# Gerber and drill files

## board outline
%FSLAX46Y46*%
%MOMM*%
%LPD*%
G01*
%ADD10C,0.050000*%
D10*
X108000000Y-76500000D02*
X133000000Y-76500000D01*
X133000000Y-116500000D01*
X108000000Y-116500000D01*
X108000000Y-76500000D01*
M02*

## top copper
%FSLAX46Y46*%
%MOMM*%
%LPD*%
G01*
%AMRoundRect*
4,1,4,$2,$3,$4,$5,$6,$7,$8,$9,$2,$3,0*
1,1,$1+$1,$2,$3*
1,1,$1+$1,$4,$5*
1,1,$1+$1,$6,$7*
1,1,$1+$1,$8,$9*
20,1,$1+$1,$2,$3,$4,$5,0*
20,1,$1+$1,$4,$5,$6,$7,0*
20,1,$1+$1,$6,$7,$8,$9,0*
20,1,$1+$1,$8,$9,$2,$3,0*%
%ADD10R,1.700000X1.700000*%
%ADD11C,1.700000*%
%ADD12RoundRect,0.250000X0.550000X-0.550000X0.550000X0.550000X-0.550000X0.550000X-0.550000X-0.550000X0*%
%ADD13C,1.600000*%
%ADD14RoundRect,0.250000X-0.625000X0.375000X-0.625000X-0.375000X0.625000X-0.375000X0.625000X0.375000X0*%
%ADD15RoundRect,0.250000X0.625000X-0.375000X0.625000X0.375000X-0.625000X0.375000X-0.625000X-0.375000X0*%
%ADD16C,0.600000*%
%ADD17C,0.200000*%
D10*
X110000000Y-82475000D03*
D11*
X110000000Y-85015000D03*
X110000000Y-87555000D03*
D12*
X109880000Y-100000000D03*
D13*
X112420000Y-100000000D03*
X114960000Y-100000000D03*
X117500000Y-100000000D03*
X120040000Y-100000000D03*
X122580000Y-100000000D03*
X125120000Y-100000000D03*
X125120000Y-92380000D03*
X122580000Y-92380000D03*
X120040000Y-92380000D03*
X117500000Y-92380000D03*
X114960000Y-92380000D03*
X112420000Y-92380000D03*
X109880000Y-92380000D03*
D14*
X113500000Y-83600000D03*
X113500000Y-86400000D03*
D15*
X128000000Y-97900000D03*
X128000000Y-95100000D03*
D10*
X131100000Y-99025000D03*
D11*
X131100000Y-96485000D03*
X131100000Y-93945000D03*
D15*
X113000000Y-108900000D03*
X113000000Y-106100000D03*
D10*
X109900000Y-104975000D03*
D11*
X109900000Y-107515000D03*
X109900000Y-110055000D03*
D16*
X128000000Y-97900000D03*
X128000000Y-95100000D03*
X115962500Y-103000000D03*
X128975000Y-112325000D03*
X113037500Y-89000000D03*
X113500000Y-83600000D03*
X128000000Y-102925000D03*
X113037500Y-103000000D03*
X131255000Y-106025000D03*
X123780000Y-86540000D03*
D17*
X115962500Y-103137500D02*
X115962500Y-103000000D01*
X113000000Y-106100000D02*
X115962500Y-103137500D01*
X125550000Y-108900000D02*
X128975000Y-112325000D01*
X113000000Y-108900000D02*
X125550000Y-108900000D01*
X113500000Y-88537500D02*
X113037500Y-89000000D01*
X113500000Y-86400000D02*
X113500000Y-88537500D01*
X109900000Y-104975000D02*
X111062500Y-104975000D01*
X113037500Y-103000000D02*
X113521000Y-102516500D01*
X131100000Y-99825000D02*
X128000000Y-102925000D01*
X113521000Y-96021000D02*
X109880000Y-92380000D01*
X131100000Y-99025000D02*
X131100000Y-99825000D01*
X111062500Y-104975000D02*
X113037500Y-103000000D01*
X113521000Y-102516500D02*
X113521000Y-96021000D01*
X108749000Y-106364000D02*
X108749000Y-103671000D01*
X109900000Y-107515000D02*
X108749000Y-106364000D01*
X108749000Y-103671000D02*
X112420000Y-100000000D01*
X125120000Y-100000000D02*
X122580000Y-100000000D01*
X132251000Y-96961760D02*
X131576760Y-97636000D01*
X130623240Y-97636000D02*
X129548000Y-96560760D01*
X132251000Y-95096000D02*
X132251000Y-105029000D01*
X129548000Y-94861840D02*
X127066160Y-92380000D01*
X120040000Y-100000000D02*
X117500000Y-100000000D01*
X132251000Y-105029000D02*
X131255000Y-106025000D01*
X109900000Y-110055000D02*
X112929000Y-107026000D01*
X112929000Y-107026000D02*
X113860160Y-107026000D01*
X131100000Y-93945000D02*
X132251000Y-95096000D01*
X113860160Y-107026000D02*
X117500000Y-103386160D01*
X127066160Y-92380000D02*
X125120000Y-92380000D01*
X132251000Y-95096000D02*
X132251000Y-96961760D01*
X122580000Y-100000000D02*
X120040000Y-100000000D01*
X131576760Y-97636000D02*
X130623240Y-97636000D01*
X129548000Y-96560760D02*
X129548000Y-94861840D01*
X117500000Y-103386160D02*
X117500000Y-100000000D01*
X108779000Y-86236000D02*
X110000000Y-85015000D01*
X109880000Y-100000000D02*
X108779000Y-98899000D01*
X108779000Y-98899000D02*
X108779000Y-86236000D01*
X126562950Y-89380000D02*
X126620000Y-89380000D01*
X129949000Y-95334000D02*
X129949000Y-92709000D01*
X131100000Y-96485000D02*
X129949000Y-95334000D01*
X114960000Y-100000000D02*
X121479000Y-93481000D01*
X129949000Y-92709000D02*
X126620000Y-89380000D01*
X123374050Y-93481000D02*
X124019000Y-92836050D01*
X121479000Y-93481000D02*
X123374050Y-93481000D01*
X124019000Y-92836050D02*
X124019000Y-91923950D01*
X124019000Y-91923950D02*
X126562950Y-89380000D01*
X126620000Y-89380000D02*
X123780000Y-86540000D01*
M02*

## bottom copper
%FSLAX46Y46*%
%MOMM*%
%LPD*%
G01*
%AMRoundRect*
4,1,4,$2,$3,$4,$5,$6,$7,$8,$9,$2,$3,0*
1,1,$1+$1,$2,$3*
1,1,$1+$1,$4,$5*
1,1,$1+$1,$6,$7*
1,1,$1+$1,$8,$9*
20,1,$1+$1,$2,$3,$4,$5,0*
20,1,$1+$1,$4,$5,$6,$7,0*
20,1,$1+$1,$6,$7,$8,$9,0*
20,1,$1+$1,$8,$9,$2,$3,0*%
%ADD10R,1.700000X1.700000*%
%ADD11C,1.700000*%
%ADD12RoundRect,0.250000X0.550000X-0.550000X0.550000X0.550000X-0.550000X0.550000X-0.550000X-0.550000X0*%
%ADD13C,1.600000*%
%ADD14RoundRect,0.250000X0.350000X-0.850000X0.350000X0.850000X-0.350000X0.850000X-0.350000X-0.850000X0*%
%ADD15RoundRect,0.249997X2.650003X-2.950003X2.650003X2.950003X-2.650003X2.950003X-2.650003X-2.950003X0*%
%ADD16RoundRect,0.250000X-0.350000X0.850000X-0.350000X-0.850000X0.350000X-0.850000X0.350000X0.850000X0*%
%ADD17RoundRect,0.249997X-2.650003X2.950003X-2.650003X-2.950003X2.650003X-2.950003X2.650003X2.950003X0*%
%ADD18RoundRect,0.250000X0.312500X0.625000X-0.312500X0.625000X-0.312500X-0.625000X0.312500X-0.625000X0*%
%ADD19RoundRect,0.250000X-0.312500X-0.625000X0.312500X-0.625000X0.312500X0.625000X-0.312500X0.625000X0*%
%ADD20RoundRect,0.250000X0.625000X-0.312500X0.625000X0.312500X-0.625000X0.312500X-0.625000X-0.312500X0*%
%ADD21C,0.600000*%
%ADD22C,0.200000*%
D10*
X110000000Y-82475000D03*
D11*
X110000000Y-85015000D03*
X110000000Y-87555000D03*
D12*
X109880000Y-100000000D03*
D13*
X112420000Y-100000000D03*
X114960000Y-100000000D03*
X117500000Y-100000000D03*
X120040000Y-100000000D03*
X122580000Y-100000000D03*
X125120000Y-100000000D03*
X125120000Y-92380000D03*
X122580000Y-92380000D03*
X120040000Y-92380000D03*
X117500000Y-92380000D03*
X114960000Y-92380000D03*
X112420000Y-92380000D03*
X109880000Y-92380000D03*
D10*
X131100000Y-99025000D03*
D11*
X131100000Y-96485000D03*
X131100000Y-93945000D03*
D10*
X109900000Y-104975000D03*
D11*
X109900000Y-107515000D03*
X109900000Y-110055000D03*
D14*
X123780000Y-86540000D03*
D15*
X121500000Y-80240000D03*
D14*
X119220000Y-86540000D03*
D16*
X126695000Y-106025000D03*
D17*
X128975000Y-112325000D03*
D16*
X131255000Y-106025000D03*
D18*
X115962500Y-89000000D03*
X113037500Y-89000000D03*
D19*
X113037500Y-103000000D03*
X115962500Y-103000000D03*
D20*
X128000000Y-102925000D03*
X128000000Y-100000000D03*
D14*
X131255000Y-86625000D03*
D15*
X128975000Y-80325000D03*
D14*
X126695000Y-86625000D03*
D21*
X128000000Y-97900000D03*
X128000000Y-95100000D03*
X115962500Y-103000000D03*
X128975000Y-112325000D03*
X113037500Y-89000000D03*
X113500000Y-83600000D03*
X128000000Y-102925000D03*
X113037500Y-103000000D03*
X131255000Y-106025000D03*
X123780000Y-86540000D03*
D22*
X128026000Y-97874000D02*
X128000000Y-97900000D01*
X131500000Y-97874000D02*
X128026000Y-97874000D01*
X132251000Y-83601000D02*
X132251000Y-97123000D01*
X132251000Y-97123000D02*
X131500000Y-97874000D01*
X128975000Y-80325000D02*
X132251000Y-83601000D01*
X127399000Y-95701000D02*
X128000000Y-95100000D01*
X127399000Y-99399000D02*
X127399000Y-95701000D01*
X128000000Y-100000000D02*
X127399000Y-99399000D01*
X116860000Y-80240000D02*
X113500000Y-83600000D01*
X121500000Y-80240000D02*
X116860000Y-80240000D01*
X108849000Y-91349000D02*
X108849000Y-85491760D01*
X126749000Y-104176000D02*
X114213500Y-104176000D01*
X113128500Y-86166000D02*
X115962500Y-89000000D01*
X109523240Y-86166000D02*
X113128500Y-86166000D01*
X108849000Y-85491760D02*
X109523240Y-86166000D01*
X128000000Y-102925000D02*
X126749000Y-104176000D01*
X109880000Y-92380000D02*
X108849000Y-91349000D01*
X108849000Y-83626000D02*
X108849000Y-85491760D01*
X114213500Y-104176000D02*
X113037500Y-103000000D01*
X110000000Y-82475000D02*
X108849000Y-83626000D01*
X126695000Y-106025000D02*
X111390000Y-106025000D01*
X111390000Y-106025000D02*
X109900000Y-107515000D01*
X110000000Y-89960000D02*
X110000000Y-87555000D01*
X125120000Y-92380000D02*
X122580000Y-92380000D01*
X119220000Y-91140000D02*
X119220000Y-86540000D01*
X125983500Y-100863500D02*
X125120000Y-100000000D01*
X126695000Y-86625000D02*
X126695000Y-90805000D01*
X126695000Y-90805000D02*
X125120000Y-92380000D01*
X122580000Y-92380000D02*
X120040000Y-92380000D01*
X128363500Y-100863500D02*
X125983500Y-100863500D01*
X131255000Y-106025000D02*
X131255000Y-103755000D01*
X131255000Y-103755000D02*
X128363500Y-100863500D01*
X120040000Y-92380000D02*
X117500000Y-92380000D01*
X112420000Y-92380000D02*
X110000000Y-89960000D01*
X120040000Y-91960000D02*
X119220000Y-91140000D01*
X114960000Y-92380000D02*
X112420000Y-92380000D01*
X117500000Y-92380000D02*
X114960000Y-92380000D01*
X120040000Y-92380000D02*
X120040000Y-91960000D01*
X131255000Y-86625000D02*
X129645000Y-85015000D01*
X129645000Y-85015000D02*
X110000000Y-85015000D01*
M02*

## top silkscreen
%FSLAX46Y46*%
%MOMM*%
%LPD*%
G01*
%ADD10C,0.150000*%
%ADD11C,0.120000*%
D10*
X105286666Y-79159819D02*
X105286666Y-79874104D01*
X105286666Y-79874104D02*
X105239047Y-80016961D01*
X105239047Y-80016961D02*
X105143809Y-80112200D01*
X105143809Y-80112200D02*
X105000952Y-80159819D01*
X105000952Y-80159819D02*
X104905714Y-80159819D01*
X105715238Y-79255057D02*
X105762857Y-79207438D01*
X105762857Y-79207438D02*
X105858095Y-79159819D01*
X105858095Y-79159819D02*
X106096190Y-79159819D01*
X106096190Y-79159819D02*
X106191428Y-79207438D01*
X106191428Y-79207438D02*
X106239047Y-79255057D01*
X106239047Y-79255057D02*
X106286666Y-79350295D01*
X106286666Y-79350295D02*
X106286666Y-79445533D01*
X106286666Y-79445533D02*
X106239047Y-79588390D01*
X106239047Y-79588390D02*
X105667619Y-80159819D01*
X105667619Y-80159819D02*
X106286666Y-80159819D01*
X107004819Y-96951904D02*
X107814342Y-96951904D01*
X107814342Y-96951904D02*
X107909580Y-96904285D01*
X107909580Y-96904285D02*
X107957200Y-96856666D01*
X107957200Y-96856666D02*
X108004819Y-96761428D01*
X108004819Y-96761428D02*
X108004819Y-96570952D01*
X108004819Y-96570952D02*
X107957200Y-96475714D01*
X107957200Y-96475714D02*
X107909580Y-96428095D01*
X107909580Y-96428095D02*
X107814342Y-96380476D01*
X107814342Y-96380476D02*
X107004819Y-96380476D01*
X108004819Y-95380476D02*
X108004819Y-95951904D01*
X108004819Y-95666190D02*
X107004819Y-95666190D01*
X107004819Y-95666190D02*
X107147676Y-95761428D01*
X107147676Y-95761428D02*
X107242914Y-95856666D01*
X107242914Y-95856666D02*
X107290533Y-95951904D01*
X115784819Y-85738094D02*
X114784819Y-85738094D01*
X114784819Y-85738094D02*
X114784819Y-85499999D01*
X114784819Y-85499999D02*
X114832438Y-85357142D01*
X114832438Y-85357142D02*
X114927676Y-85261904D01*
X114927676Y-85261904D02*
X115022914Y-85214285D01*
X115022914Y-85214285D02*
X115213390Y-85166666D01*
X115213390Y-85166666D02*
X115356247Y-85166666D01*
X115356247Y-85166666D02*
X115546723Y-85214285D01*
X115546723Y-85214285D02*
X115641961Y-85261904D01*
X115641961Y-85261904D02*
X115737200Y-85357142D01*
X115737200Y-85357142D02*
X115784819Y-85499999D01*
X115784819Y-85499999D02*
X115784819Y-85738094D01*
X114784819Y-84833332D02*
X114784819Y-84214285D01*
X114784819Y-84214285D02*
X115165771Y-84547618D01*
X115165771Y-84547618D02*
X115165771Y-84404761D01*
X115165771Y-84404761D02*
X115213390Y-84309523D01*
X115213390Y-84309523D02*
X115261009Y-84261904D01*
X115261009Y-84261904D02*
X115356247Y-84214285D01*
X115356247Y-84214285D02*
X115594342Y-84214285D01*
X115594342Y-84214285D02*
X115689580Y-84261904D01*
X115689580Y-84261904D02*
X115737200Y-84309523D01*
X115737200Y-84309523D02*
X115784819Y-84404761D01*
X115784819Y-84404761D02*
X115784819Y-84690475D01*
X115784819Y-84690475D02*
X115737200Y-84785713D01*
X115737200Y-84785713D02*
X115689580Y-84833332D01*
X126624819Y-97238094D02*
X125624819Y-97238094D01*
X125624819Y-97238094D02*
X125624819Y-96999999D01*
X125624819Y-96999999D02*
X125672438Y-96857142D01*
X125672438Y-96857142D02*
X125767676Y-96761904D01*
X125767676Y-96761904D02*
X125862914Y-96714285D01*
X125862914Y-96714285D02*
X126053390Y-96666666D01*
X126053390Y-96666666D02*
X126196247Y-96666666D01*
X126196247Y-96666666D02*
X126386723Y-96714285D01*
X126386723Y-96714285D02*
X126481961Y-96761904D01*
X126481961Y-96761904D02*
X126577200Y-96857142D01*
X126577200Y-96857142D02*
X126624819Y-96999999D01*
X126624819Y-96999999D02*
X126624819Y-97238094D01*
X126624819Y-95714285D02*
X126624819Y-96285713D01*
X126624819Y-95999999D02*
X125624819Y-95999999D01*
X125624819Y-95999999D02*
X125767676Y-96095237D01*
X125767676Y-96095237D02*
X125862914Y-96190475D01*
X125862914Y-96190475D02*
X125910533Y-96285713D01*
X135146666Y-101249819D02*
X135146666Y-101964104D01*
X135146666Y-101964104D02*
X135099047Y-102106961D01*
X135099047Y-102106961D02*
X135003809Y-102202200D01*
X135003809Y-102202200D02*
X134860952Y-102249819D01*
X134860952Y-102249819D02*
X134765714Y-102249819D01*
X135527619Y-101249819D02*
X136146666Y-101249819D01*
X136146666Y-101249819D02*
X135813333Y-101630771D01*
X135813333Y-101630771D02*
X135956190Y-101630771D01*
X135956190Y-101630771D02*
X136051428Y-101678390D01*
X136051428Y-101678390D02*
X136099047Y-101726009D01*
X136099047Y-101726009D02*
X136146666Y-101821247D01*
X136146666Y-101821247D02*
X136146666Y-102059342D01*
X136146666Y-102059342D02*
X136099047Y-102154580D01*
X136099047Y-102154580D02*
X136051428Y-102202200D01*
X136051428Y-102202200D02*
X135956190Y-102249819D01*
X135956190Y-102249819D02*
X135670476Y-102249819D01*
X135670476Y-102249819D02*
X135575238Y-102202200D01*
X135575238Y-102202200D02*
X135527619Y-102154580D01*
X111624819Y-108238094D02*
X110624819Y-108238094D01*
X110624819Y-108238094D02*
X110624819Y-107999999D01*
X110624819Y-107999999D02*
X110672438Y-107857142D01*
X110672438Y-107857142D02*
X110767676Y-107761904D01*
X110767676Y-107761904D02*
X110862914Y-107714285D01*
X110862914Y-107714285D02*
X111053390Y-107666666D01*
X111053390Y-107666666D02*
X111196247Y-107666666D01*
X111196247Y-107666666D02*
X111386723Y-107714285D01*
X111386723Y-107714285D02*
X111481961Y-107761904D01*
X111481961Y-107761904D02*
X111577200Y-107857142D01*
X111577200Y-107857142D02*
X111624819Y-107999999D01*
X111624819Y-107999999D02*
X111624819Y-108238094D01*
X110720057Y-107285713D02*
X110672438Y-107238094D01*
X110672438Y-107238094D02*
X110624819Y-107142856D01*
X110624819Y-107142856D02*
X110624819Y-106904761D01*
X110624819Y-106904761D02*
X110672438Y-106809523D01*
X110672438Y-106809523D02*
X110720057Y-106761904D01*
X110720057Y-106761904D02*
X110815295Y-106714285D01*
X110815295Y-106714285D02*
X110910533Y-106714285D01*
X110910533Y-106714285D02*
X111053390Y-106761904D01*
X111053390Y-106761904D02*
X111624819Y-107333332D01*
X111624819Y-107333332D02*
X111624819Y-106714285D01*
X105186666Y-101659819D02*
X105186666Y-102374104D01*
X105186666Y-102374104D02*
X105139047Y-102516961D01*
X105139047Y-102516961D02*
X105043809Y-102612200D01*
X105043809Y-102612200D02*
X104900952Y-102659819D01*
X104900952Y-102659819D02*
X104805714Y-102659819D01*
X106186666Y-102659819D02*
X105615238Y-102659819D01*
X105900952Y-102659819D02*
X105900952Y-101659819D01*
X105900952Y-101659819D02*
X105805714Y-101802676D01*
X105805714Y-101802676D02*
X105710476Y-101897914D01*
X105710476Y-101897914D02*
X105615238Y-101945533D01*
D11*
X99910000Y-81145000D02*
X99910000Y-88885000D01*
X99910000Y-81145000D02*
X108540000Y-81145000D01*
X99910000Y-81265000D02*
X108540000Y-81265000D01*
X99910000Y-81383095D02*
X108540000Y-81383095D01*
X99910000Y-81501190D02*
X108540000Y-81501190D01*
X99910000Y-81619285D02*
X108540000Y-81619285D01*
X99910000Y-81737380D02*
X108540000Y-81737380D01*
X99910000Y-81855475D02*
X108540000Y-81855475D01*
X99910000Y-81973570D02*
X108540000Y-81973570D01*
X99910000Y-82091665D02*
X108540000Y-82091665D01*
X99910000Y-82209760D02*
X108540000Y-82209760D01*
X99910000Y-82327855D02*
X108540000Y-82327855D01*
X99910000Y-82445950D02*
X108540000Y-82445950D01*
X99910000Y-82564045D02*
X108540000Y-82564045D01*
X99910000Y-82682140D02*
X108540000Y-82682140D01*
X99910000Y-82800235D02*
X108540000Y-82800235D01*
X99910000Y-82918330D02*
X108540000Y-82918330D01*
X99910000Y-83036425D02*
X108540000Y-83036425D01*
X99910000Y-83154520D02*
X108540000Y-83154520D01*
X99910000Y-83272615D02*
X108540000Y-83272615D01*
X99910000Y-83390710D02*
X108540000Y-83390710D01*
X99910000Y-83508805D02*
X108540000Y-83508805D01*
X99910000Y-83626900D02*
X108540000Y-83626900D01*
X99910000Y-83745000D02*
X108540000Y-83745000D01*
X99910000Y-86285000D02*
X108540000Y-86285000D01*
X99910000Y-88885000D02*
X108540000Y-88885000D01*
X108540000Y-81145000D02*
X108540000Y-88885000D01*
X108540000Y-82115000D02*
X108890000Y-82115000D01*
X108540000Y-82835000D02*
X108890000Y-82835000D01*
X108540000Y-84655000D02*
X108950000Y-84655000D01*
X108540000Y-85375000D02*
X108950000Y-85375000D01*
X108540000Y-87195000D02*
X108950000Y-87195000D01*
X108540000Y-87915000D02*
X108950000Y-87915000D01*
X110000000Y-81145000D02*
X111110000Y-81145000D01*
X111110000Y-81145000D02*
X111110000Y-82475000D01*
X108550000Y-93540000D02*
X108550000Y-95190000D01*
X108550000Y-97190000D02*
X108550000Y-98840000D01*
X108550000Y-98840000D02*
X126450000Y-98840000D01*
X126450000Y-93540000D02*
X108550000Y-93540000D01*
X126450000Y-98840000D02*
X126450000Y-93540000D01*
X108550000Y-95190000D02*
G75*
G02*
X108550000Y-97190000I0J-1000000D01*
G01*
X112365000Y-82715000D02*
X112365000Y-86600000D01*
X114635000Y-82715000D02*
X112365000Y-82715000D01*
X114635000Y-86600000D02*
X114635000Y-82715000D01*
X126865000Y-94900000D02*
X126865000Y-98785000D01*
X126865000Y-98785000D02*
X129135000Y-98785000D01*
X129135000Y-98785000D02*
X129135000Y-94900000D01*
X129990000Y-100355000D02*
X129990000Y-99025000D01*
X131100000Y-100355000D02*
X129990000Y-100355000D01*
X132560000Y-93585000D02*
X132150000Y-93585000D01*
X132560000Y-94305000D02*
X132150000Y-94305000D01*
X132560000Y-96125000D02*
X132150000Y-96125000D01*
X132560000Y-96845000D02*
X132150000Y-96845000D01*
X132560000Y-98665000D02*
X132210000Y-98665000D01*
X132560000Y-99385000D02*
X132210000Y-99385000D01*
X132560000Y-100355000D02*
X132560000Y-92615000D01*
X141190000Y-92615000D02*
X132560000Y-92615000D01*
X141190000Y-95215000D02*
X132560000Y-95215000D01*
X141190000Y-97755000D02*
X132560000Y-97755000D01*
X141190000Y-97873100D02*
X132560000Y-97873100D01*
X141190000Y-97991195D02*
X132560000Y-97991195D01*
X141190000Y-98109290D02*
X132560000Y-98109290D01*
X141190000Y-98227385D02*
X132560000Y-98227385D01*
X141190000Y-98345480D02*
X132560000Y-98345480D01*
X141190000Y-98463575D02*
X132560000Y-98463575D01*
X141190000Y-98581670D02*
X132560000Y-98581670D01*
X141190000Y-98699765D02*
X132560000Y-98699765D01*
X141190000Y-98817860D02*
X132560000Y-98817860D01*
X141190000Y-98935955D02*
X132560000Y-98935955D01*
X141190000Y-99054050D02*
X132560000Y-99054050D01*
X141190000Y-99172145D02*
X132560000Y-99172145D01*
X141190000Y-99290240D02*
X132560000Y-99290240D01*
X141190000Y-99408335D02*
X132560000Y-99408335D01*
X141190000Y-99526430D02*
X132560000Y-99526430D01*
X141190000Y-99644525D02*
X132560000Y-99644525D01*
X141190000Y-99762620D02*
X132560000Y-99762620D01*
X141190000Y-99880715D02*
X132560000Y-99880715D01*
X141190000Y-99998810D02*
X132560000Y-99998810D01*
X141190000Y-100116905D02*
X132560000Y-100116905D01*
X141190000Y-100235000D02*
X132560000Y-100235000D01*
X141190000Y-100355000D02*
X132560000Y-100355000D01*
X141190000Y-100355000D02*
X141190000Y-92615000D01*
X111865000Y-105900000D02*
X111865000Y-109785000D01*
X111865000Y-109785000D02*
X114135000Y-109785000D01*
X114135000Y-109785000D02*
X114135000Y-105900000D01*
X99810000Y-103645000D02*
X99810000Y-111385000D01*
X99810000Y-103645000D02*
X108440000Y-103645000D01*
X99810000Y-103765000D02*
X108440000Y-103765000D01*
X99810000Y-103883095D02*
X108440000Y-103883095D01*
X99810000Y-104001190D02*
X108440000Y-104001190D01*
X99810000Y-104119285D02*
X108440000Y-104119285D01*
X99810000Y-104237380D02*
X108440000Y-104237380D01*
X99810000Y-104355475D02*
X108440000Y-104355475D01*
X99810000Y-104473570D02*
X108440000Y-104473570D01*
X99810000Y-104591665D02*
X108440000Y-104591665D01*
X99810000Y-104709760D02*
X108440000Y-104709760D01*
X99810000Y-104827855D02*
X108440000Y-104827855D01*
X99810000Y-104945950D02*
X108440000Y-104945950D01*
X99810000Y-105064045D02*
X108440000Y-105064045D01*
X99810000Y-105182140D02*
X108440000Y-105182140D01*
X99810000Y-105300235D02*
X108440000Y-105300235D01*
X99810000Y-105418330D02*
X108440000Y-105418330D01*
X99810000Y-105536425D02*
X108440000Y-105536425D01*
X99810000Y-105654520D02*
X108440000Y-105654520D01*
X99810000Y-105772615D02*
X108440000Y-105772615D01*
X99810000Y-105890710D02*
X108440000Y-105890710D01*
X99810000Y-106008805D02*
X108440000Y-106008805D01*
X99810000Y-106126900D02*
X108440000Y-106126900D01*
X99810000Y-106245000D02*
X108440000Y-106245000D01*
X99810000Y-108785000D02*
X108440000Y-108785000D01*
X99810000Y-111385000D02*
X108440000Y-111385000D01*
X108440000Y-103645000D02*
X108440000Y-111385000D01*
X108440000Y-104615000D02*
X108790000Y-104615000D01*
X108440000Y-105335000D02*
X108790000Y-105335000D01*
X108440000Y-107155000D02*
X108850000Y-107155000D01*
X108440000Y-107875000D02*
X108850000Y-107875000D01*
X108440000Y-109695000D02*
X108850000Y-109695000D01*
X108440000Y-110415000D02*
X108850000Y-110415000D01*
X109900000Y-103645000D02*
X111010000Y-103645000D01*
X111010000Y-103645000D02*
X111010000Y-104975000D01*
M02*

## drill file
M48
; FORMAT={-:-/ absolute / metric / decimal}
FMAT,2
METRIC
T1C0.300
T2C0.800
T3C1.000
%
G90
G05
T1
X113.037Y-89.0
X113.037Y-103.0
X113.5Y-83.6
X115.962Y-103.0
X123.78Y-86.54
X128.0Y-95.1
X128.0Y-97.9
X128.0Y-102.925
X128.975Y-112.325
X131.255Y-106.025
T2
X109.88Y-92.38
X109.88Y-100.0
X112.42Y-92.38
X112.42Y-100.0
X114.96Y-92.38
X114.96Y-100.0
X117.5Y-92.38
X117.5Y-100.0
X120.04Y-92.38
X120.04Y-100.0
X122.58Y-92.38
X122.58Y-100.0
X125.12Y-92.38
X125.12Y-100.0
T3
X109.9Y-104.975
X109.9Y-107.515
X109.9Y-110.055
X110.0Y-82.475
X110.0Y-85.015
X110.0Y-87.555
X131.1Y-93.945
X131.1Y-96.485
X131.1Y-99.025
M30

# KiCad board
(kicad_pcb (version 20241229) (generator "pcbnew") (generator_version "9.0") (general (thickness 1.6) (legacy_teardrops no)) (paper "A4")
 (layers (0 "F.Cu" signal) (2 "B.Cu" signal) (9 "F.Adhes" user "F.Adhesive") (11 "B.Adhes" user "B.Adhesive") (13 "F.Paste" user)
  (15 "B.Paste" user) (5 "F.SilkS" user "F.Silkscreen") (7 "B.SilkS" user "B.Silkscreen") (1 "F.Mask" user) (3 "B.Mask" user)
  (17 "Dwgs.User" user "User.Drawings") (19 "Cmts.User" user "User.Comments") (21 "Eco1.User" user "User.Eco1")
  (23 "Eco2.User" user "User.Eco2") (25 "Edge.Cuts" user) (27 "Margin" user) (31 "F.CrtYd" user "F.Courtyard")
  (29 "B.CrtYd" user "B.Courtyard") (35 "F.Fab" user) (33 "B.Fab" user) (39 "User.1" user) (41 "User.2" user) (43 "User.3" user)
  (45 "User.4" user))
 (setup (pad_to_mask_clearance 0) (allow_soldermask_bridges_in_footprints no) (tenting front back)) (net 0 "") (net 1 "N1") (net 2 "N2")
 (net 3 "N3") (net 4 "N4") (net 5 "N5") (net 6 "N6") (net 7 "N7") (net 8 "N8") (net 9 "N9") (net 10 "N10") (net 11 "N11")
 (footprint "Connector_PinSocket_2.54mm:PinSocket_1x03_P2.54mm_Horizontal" (layer "F.Cu") (at 110 82.475)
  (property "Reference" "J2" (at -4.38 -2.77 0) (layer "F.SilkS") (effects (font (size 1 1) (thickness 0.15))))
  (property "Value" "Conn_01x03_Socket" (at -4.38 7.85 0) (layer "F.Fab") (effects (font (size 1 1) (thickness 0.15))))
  (fp_line (start -10.09 -1.33) (end -10.09 6.41) (stroke (width 0.12) (type solid)) (layer "F.SilkS"))
  (fp_line (start -10.09 -1.33) (end -1.46 -1.33) (stroke (width 0.12) (type solid)) (layer "F.SilkS"))
  (fp_line (start -10.09 -1.21) (end -1.46 -1.21) (stroke (width 0.12) (type solid)) (layer "F.SilkS"))
  (fp_line (start -10.09 -1.091905) (end -1.46 -1.091905) (stroke (width 0.12) (type solid)) (layer "F.SilkS"))
  (fp_line (start -10.09 -0.97381) (end -1.46 -0.97381) (stroke (width 0.12) (type solid)) (layer "F.SilkS"))
  (fp_line (start -10.09 -0.855715) (end -1.46 -0.855715) (stroke (width 0.12) (type solid)) (layer "F.SilkS"))
  (fp_line (start -10.09 -0.73762) (end -1.46 -0.73762) (stroke (width 0.12) (type solid)) (layer "F.SilkS"))
  (fp_line (start -10.09 -0.619525) (end -1.46 -0.619525) (stroke (width 0.12) (type solid)) (layer "F.SilkS"))
  (fp_line (start -10.09 -0.50143) (end -1.46 -0.50143) (stroke (width 0.12) (type solid)) (layer "F.SilkS"))
  (fp_line (start -10.09 -0.383335) (end -1.46 -0.383335) (stroke (width 0.12) (type solid)) (layer "F.SilkS"))
  (fp_line (start -10.09 -0.26524) (end -1.46 -0.26524) (stroke (width 0.12) (type solid)) (layer "F.SilkS"))
  (fp_line (start -10.09 -0.147145) (end -1.46 -0.147145) (stroke (width 0.12) (type solid)) (layer "F.SilkS"))
  (fp_line (start -10.09 -0.02905) (end -1.46 -0.02905) (stroke (width 0.12) (type solid)) (layer "F.SilkS"))
  (fp_line (start -10.09 0.089045) (end -1.46 0.089045) (stroke (width 0.12) (type solid)) (layer "F.SilkS"))
  (fp_line (start -10.09 0.20714) (end -1.46 0.20714) (stroke (width 0.12) (type solid)) (layer "F.SilkS"))
  (fp_line (start -10.09 0.325235) (end -1.46 0.325235) (stroke (width 0.12) (type solid)) (layer "F.SilkS"))
  (fp_line (start -10.09 0.44333) (end -1.46 0.44333) (stroke (width 0.12) (type solid)) (layer "F.SilkS"))
  (fp_line (start -10.09 0.561425) (end -1.46 0.561425) (stroke (width 0.12) (type solid)) (layer "F.SilkS"))
  (fp_line (start -10.09 0.67952) (end -1.46 0.67952) (stroke (width 0.12) (type solid)) (layer "F.SilkS"))
  (fp_line (start -10.09 0.797615) (end -1.46 0.797615) (stroke (width 0.12) (type solid)) (layer "F.SilkS"))
  (fp_line (start -10.09 0.91571) (end -1.46 0.91571) (stroke (width 0.12) (type solid)) (layer "F.SilkS"))
  (fp_line (start -10.09 1.033805) (end -1.46 1.033805) (stroke (width 0.12) (type solid)) (layer "F.SilkS"))
  (fp_line (start -10.09 1.1519) (end -1.46 1.1519) (stroke (width 0.12) (type solid)) (layer "F.SilkS"))
  (fp_line (start -10.09 1.27) (end -1.46 1.27) (stroke (width 0.12) (type solid)) (layer "F.SilkS"))
  (fp_line (start -10.09 3.81) (end -1.46 3.81) (stroke (width 0.12) (type solid)) (layer "F.SilkS"))
  (fp_line (start -10.09 6.41) (end -1.46 6.41) (stroke (width 0.12) (type solid)) (layer "F.SilkS"))
  (fp_line (start -1.46 -1.33) (end -1.46 6.41) (stroke (width 0.12) (type solid)) (layer "F.SilkS"))
  (fp_line (start -1.46 -0.36) (end -1.11 -0.36) (stroke (width 0.12) (type solid)) (layer "F.SilkS"))
  (fp_line (start -1.46 0.36) (end -1.11 0.36) (stroke (width 0.12) (type solid)) (layer "F.SilkS"))
  (fp_line (start -1.46 2.18) (end -1.05 2.18) (stroke (width 0.12) (type solid)) (layer "F.SilkS"))
  (fp_line (start -1.46 2.9) (end -1.05 2.9) (stroke (width 0.12) (type solid)) (layer "F.SilkS"))
  (fp_line (start -1.46 4.72) (end -1.05 4.72) (stroke (width 0.12) (type solid)) (layer "F.SilkS"))
  (fp_line (start -1.46 5.44) (end -1.05 5.44) (stroke (width 0.12) (type solid)) (layer "F.SilkS"))
  (fp_line (start 0 -1.33) (end 1.11 -1.33) (stroke (width 0.12) (type solid)) (layer "F.SilkS"))
  (fp_line (start 1.11 -1.33) (end 1.11 0) (stroke (width 0.12) (type solid)) (layer "F.SilkS"))
  (pad "1" thru_hole rect (at 0 0) (size 1.7 1.7) (drill 1) (layers "*.Cu" "*.Mask") (remove_unused_layers no) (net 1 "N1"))
  (pad "2" thru_hole circle (at 0 2.54) (size 1.7 1.7) (drill 1) (layers "*.Cu" "*.Mask") (remove_unused_layers no) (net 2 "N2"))
  (pad "3" thru_hole circle (at 0 5.08) (size 1.7 1.7) (drill 1) (layers "*.Cu" "*.Mask") (remove_unused_layers no) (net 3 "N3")))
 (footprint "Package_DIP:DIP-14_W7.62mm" (layer "F.Cu") (at 109.88 100 90)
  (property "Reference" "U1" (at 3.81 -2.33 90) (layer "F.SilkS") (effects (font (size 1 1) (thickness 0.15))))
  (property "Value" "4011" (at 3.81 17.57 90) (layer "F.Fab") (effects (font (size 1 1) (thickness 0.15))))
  (fp_line (start 6.46 -1.33) (end 4.81 -1.33) (stroke (width 0.12) (type solid)) (layer "F.SilkS"))
  (fp_line (start 2.81 -1.33) (end 1.16 -1.33) (stroke (width 0.12) (type solid)) (layer "F.SilkS"))
  (fp_line (start 1.16 -1.33) (end 1.16 16.57) (stroke (width 0.12) (type solid)) (layer "F.SilkS"))
  (fp_line (start 6.46 16.57) (end 6.46 -1.33) (stroke (width 0.12) (type solid)) (layer "F.SilkS"))
  (fp_line (start 1.16 16.57) (end 6.46 16.57) (stroke (width 0.12) (type solid)) (layer "F.SilkS"))
  (fp_arc (start 4.81 -1.33) (mid 3.81 -0.33) (end 2.81 -1.33) (stroke (width 0.12) (type solid)) (layer "F.SilkS"))
  (pad "1" thru_hole roundrect (at 0 0 90) (size 1.6 1.6) (drill 0.8) (layers "*.Cu" "*.Mask") (remove_unused_layers no)
   (roundrect_rratio 0.15625) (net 2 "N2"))
  (pad "2" thru_hole circle (at 0 2.54 90) (size 1.6 1.6) (drill 0.8) (layers "*.Cu" "*.Mask") (remove_unused_layers no) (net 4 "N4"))
  (pad "3" thru_hole circle (at 0 5.08 90) (size 1.6 1.6) (drill 0.8) (layers "*.Cu" "*.Mask") (remove_unused_layers no) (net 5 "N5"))
  (pad "4" thru_hole circle (at 0 7.62 90) (size 1.6 1.6) (drill 0.8) (layers "*.Cu" "*.Mask") (remove_unused_layers no) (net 3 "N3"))
  (pad "5" thru_hole circle (at 0 10.16 90) (size 1.6 1.6) (drill 0.8) (layers "*.Cu" "*.Mask") (remove_unused_layers no) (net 3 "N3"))
  (pad "6" thru_hole circle (at 0 12.7 90) (size 1.6 1.6) (drill 0.8) (layers "*.Cu" "*.Mask") (remove_unused_layers no) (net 3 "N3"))
  (pad "7" thru_hole circle (at 0 15.24 90) (size 1.6 1.6) (drill 0.8) (layers "*.Cu" "*.Mask") (remove_unused_layers no) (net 3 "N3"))
  (pad "8" thru_hole circle (at 7.62 15.24 90) (size 1.6 1.6) (drill 0.8) (layers "*.Cu" "*.Mask") (remove_unused_layers no) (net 3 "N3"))
  (pad "9" thru_hole circle (at 7.62 12.7 90) (size 1.6 1.6) (drill 0.8) (layers "*.Cu" "*.Mask") (remove_unused_layers no) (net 3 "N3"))
  (pad "10" thru_hole circle (at 7.62 10.16 90) (size 1.6 1.6) (drill 0.8) (layers "*.Cu" "*.Mask") (remove_unused_layers no) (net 3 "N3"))
  (pad "11" thru_hole circle (at 7.62 7.62 90) (size 1.6 1.6) (drill 0.8) (layers "*.Cu" "*.Mask") (remove_unused_layers no) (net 3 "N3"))
  (pad "12" thru_hole circle (at 7.62 5.08 90) (size 1.6 1.6) (drill 0.8) (layers "*.Cu" "*.Mask") (remove_unused_layers no) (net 3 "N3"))
  (pad "13" thru_hole circle (at 7.62 2.54 90) (size 1.6 1.6) (drill 0.8) (layers "*.Cu" "*.Mask") (remove_unused_layers no) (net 3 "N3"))
  (pad "14" thru_hole circle (at 7.62 0 90) (size 1.6 1.6) (drill 0.8) (layers "*.Cu" "*.Mask") (remove_unused_layers no) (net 1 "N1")))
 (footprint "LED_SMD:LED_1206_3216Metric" (layer "F.Cu") (at 113.5 85 -90)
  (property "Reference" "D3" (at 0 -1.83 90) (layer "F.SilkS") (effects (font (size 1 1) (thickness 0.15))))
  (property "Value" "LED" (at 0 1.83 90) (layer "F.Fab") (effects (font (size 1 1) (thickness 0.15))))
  (fp_line (start -2.285 1.135) (end 1.6 1.135) (stroke (width 0.12) (type solid)) (layer "F.SilkS"))
  (fp_line (start -2.285 -1.135) (end -2.285 1.135) (stroke (width 0.12) (type solid)) (layer "F.SilkS"))
  (fp_line (start 1.6 -1.135) (end -2.285 -1.135) (stroke (width 0.12) (type solid)) (layer "F.SilkS"))
  (pad "1" smd roundrect (at -1.4 0 270) (size 1.25 1.75) (layers "F.Cu" "F.Mask" "F.Paste") (roundrect_rratio 0.2) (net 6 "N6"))
  (pad "2" smd roundrect (at 1.4 0 270) (size 1.25 1.75) (layers "F.Cu" "F.Mask" "F.Paste") (roundrect_rratio 0.2) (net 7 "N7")))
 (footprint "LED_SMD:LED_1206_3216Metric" (layer "F.Cu") (at 128 96.5 90)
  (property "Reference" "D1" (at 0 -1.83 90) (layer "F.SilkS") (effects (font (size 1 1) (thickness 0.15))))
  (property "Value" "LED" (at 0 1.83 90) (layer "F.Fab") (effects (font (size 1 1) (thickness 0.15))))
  (fp_line (start 1.6 -1.135) (end -2.285 -1.135) (stroke (width 0.12) (type solid)) (layer "F.SilkS"))
  (fp_line (start -2.285 -1.135) (end -2.285 1.135) (stroke (width 0.12) (type solid)) (layer "F.SilkS"))
  (fp_line (start -2.285 1.135) (end 1.6 1.135) (stroke (width 0.12) (type solid)) (layer "F.SilkS"))
  (pad "1" smd roundrect (at -1.4 0 90) (size 1.25 1.75) (layers "F.Cu" "F.Mask" "F.Paste") (roundrect_rratio 0.2) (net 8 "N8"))
  (pad "2" smd roundrect (at 1.4 0 90) (size 1.25 1.75) (layers "F.Cu" "F.Mask" "F.Paste") (roundrect_rratio 0.2) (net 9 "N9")))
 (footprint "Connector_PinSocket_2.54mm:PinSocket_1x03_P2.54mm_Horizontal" (layer "F.Cu") (at 131.1 99.025 180)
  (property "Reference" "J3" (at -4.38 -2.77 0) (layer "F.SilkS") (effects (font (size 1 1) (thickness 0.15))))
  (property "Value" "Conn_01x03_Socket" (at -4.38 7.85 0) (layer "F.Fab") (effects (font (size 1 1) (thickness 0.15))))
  (fp_line (start 1.11 -1.33) (end 1.11 0) (stroke (width 0.12) (type solid)) (layer "F.SilkS"))
  (fp_line (start 0 -1.33) (end 1.11 -1.33) (stroke (width 0.12) (type solid)) (layer "F.SilkS"))
  (fp_line (start -1.46 5.44) (end -1.05 5.44) (stroke (width 0.12) (type solid)) (layer "F.SilkS"))
  (fp_line (start -1.46 4.72) (end -1.05 4.72) (stroke (width 0.12) (type solid)) (layer "F.SilkS"))
  (fp_line (start -1.46 2.9) (end -1.05 2.9) (stroke (width 0.12) (type solid)) (layer "F.SilkS"))
  (fp_line (start -1.46 2.18) (end -1.05 2.18) (stroke (width 0.12) (type solid)) (layer "F.SilkS"))
  (fp_line (start -1.46 0.36) (end -1.11 0.36) (stroke (width 0.12) (type solid)) (layer "F.SilkS"))
  (fp_line (start -1.46 -0.36) (end -1.11 -0.36) (stroke (width 0.12) (type solid)) (layer "F.SilkS"))
  (fp_line (start -1.46 -1.33) (end -1.46 6.41) (stroke (width 0.12) (type solid)) (layer "F.SilkS"))
  (fp_line (start -10.09 6.41) (end -1.46 6.41) (stroke (width 0.12) (type solid)) (layer "F.SilkS"))
  (fp_line (start -10.09 3.81) (end -1.46 3.81) (stroke (width 0.12) (type solid)) (layer "F.SilkS"))
  (fp_line (start -10.09 1.27) (end -1.46 1.27) (stroke (width 0.12) (type solid)) (layer "F.SilkS"))
  (fp_line (start -10.09 1.1519) (end -1.46 1.1519) (stroke (width 0.12) (type solid)) (layer "F.SilkS"))
  (fp_line (start -10.09 1.033805) (end -1.46 1.033805) (stroke (width 0.12) (type solid)) (layer "F.SilkS"))
  (fp_line (start -10.09 0.91571) (end -1.46 0.91571) (stroke (width 0.12) (type solid)) (layer "F.SilkS"))
  (fp_line (start -10.09 0.797615) (end -1.46 0.797615) (stroke (width 0.12) (type solid)) (layer "F.SilkS"))
  (fp_line (start -10.09 0.67952) (end -1.46 0.67952) (stroke (width 0.12) (type solid)) (layer "F.SilkS"))
  (fp_line (start -10.09 0.561425) (end -1.46 0.561425) (stroke (width 0.12) (type solid)) (layer "F.SilkS"))
  (fp_line (start -10.09 0.44333) (end -1.46 0.44333) (stroke (width 0.12) (type solid)) (layer "F.SilkS"))
  (fp_line (start -10.09 0.325235) (end -1.46 0.325235) (stroke (width 0.12) (type solid)) (layer "F.SilkS"))
  (fp_line (start -10.09 0.20714) (end -1.46 0.20714) (stroke (width 0.12) (type solid)) (layer "F.SilkS"))
  (fp_line (start -10.09 0.089045) (end -1.46 0.089045) (stroke (width 0.12) (type solid)) (layer "F.SilkS"))
  (fp_line (start -10.09 -0.02905) (end -1.46 -0.02905) (stroke (width 0.12) (type solid)) (layer "F.SilkS"))
  (fp_line (start -10.09 -0.147145) (end -1.46 -0.147145) (stroke (width 0.12) (type solid)) (layer "F.SilkS"))
  (fp_line (start -10.09 -0.26524) (end -1.46 -0.26524) (stroke (width 0.12) (type solid)) (layer "F.SilkS"))
  (fp_line (start -10.09 -0.383335) (end -1.46 -0.383335) (stroke (width 0.12) (type solid)) (layer "F.SilkS"))
  (fp_line (start -10.09 -0.50143) (end -1.46 -0.50143) (stroke (width 0.12) (type solid)) (layer "F.SilkS"))
  (fp_line (start -10.09 -0.619525) (end -1.46 -0.619525) (stroke (width 0.12) (type solid)) (layer "F.SilkS"))
  (fp_line (start -10.09 -0.73762) (end -1.46 -0.73762) (stroke (width 0.12) (type solid)) (layer "F.SilkS"))
  (fp_line (start -10.09 -0.855715) (end -1.46 -0.855715) (stroke (width 0.12) (type solid)) (layer "F.SilkS"))
  (fp_line (start -10.09 -0.97381) (end -1.46 -0.97381) (stroke (width 0.12) (type solid)) (layer "F.SilkS"))
  (fp_line (start -10.09 -1.091905) (end -1.46 -1.091905) (stroke (width 0.12) (type solid)) (layer "F.SilkS"))
  (fp_line (start -10.09 -1.21) (end -1.46 -1.21) (stroke (width 0.12) (type solid)) (layer "F.SilkS"))
  (fp_line (start -10.09 -1.33) (end -1.46 -1.33) (stroke (width 0.12) (type solid)) (layer "F.SilkS"))
  (fp_line (start -10.09 -1.33) (end -10.09 6.41) (stroke (width 0.12) (type solid)) (layer "F.SilkS"))
  (pad "1" thru_hole rect (at 0 0 180) (size 1.7 1.7) (drill 1) (layers "*.Cu" "*.Mask") (remove_unused_layers no) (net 1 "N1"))
  (pad "2" thru_hole circle (at 0 2.54 180) (size 1.7 1.7) (drill 1) (layers "*.Cu" "*.Mask") (remove_unused_layers no) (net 5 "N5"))
  (pad "3" thru_hole circle (at 0 5.08 180) (size 1.7 1.7) (drill 1) (layers "*.Cu" "*.Mask") (remove_unused_layers no) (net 3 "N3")))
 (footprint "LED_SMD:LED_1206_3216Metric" (layer "F.Cu") (at 113 107.5 90)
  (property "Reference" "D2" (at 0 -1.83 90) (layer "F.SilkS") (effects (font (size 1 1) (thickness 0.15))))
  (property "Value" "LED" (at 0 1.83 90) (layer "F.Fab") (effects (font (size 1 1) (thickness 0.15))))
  (fp_line (start 1.6 -1.135) (end -2.285 -1.135) (stroke (width 0.12) (type solid)) (layer "F.SilkS"))
  (fp_line (start -2.285 -1.135) (end -2.285 1.135) (stroke (width 0.12) (type solid)) (layer "F.SilkS"))
  (fp_line (start -2.285 1.135) (end 1.6 1.135) (stroke (width 0.12) (type solid)) (layer "F.SilkS"))
  (pad "1" smd roundrect (at -1.4 0 90) (size 1.25 1.75) (layers "F.Cu" "F.Mask" "F.Paste") (roundrect_rratio 0.2) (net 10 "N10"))
  (pad "2" smd roundrect (at 1.4 0 90) (size 1.25 1.75) (layers "F.Cu" "F.Mask" "F.Paste") (roundrect_rratio 0.2) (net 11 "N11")))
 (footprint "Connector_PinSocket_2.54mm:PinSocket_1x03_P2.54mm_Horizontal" (layer "F.Cu") (at 109.9 104.975)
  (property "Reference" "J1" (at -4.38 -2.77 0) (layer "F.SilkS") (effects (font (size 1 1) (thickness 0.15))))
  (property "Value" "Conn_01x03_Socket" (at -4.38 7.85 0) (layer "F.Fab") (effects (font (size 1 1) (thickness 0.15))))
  (fp_line (start -10.09 -1.33) (end -10.09 6.41) (stroke (width 0.12) (type solid)) (layer "F.SilkS"))
  (fp_line (start -10.09 -1.33) (end -1.46 -1.33) (stroke (width 0.12) (type solid)) (layer "F.SilkS"))
  (fp_line (start -10.09 -1.21) (end -1.46 -1.21) (stroke (width 0.12) (type solid)) (layer "F.SilkS"))
  (fp_line (start -10.09 -1.091905) (end -1.46 -1.091905) (stroke (width 0.12) (type solid)) (layer "F.SilkS"))
  (fp_line (start -10.09 -0.97381) (end -1.46 -0.97381) (stroke (width 0.12) (type solid)) (layer "F.SilkS"))
  (fp_line (start -10.09 -0.855715) (end -1.46 -0.855715) (stroke (width 0.12) (type solid)) (layer "F.SilkS"))
  (fp_line (start -10.09 -0.73762) (end -1.46 -0.73762) (stroke (width 0.12) (type solid)) (layer "F.SilkS"))
  (fp_line (start -10.09 -0.619525) (end -1.46 -0.619525) (stroke (width 0.12) (type solid)) (layer "F.SilkS"))
  (fp_line (start -10.09 -0.50143) (end -1.46 -0.50143) (stroke (width 0.12) (type solid)) (layer "F.SilkS"))
  (fp_line (start -10.09 -0.383335) (end -1.46 -0.383335) (stroke (width 0.12) (type solid)) (layer "F.SilkS"))
  (fp_line (start -10.09 -0.26524) (end -1.46 -0.26524) (stroke (width 0.12) (type solid)) (layer "F.SilkS"))
  (fp_line (start -10.09 -0.147145) (end -1.46 -0.147145) (stroke (width 0.12) (type solid)) (layer "F.SilkS"))
  (fp_line (start -10.09 -0.02905) (end -1.46 -0.02905) (stroke (width 0.12) (type solid)) (layer "F.SilkS"))
  (fp_line (start -10.09 0.089045) (end -1.46 0.089045) (stroke (width 0.12) (type solid)) (layer "F.SilkS"))
  (fp_line (start -10.09 0.20714) (end -1.46 0.20714) (stroke (width 0.12) (type solid)) (layer "F.SilkS"))
  (fp_line (start -10.09 0.325235) (end -1.46 0.325235) (stroke (width 0.12) (type solid)) (layer "F.SilkS"))
  (fp_line (start -10.09 0.44333) (end -1.46 0.44333) (stroke (width 0.12) (type solid)) (layer "F.SilkS"))
  (fp_line (start -10.09 0.561425) (end -1.46 0.561425) (stroke (width 0.12) (type solid)) (layer "F.SilkS"))
  (fp_line (start -10.09 0.67952) (end -1.46 0.67952) (stroke (width 0.12) (type solid)) (layer "F.SilkS"))
  (fp_line (start -10.09 0.797615) (end -1.46 0.797615) (stroke (width 0.12) (type solid)) (layer "F.SilkS"))
  (fp_line (start -10.09 0.91571) (end -1.46 0.91571) (stroke (width 0.12) (type solid)) (layer "F.SilkS"))
  (fp_line (start -10.09 1.033805) (end -1.46 1.033805) (stroke (width 0.12) (type solid)) (layer "F.SilkS"))
  (fp_line (start -10.09 1.1519) (end -1.46 1.1519) (stroke (width 0.12) (type solid)) (layer "F.SilkS"))
  (fp_line (start -10.09 1.27) (end -1.46 1.27) (stroke (width 0.12) (type solid)) (layer "F.SilkS"))
  (fp_line (start -10.09 3.81) (end -1.46 3.81) (stroke (width 0.12) (type solid)) (layer "F.SilkS"))
  (fp_line (start -10.09 6.41) (end -1.46 6.41) (stroke (width 0.12) (type solid)) (layer "F.SilkS"))
  (fp_line (start -1.46 -1.33) (end -1.46 6.41) (stroke (width 0.12) (type solid)) (layer "F.SilkS"))
  (fp_line (start -1.46 -0.36) (end -1.11 -0.36) (stroke (width 0.12) (type solid)) (layer "F.SilkS"))
  (fp_line (start -1.46 0.36) (end -1.11 0.36) (stroke (width 0.12) (type solid)) (layer "F.SilkS"))
  (fp_line (start -1.46 2.18) (end -1.05 2.18) (stroke (width 0.12) (type solid)) (layer "F.SilkS"))
  (fp_line (start -1.46 2.9) (end -1.05 2.9) (stroke (width 0.12) (type solid)) (layer "F.SilkS"))
  (fp_line (start -1.46 4.72) (end -1.05 4.72) (stroke (width 0.12) (type solid)) (layer "F.SilkS"))
  (fp_line (start -1.46 5.44) (end -1.05 5.44) (stroke (width 0.12) (type solid)) (layer "F.SilkS"))
  (fp_line (start 0 -1.33) (end 1.11 -1.33) (stroke (width 0.12) (type solid)) (layer "F.SilkS"))
  (fp_line (start 1.11 -1.33) (end 1.11 0) (stroke (width 0.12) (type solid)) (layer "F.SilkS"))
  (pad "1" thru_hole rect (at 0 0) (size 1.7 1.7) (drill 1) (layers "*.Cu" "*.Mask") (remove_unused_layers no) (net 1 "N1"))
  (pad "2" thru_hole circle (at 0 2.54) (size 1.7 1.7) (drill 1) (layers "*.Cu" "*.Mask") (remove_unused_layers no) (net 4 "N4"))
  (pad "3" thru_hole circle (at 0 5.08) (size 1.7 1.7) (drill 1) (layers "*.Cu" "*.Mask") (remove_unused_layers no) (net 3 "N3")))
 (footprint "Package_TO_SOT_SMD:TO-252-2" (layer "B.Cu") (at 121.5 81.5 90)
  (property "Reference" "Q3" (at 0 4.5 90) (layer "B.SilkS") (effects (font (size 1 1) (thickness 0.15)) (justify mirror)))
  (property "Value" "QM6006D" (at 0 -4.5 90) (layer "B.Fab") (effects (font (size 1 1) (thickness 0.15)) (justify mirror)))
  (pad "" smd roundrect (at -0.415 -1.525 90) (size 3.05 2.75) (layers "B.Paste") (roundrect_rratio 0.090909))
  (pad "" smd roundrect (at -0.415 1.525 90) (size 3.05 2.75) (layers "B.Paste") (roundrect_rratio 0.090909))
  (pad "" smd roundrect (at 2.935 -1.525 90) (size 3.05 2.75) (layers "B.Paste") (roundrect_rratio 0.090909))
  (pad "" smd roundrect (at 2.935 1.525 90) (size 3.05 2.75) (layers "B.Paste") (roundrect_rratio 0.090909))
  (pad "1" smd roundrect (at -5.04 2.28 90) (size 2.2 1.2) (layers "B.Cu" "B.Mask" "B.Paste") (roundrect_rratio 0.208333) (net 5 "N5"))
  (pad "2" smd roundrect (at 1.26 0 90) (size 6.4 5.8) (layers "B.Cu" "B.Mask") (roundrect_rratio 0.043103) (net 6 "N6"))
  (pad "3" smd roundrect (at -5.04 -2.28 90) (size 2.2 1.2) (layers "B.Cu" "B.Mask" "B.Paste") (roundrect_rratio 0.208333) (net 3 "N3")))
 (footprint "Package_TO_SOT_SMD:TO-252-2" (layer "B.Cu") (at 128.975 111.065 -90)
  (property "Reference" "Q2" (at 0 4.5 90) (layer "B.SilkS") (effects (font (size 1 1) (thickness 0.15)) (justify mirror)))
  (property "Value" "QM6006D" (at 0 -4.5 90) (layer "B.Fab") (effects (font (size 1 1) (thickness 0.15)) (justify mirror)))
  (pad "" smd roundrect (at -0.415 -1.525 270) (size 3.05 2.75) (layers "B.Paste") (roundrect_rratio 0.090909))
  (pad "" smd roundrect (at -0.415 1.525 270) (size 3.05 2.75) (layers "B.Paste") (roundrect_rratio 0.090909))
  (pad "" smd roundrect (at 2.935 -1.525 270) (size 3.05 2.75) (layers "B.Paste") (roundrect_rratio 0.090909))
  (pad "" smd roundrect (at 2.935 1.525 270) (size 3.05 2.75) (layers "B.Paste") (roundrect_rratio 0.090909))
  (pad "1" smd roundrect (at -5.04 2.28 270) (size 2.2 1.2) (layers "B.Cu" "B.Mask" "B.Paste") (roundrect_rratio 0.208333) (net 4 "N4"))
  (pad "2" smd roundrect (at 1.26 0 270) (size 6.4 5.8) (layers "B.Cu" "B.Mask") (roundrect_rratio 0.043103) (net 10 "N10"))
  (pad "3" smd roundrect (at -5.04 -2.28 270) (size 2.2 1.2) (layers "B.Cu" "B.Mask" "B.Paste") (roundrect_rratio 0.208333) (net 3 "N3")))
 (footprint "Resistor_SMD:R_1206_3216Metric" (layer "B.Cu") (at 114.5 89 180)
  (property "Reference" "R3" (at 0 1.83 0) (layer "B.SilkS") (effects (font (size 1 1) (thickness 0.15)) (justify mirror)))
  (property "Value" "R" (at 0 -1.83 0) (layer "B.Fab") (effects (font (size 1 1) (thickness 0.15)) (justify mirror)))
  (pad "1" smd roundrect (at -1.4625 0 180) (size 1.125 1.75) (layers "B.Cu" "B.Mask" "B.Paste") (roundrect_rratio 0.222222) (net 1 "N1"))
  (pad "2" smd roundrect (at 1.4625 0 180) (size 1.125 1.75) (layers "B.Cu" "B.Mask" "B.Paste") (roundrect_rratio 0.222222) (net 7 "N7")))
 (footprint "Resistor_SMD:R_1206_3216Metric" (layer "B.Cu") (at 114.5 103)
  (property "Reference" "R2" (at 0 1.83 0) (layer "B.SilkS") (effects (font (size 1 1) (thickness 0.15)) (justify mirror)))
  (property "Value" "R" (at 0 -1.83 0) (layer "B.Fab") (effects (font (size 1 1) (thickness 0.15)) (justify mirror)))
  (pad "1" smd roundrect (at -1.4625 0) (size 1.125 1.75) (layers "B.Cu" "B.Mask" "B.Paste") (roundrect_rratio 0.222222) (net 1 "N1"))
  (pad "2" smd roundrect (at 1.4625 0) (size 1.125 1.75) (layers "B.Cu" "B.Mask" "B.Paste") (roundrect_rratio 0.222222) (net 11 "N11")))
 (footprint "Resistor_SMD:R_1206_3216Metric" (layer "B.Cu") (at 128 101.4625 90)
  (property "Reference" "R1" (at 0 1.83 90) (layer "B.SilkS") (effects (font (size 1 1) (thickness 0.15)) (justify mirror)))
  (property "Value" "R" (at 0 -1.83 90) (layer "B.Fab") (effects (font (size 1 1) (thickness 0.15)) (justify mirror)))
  (pad "1" smd roundrect (at -1.4625 0 90) (size 1.125 1.75) (layers "B.Cu" "B.Mask" "B.Paste") (roundrect_rratio 0.222222) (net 1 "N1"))
  (pad "2" smd roundrect (at 1.4625 0 90) (size 1.125 1.75) (layers "B.Cu" "B.Mask" "B.Paste") (roundrect_rratio 0.222222) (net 9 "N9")))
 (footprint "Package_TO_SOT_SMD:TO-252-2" (layer "B.Cu") (at 128.975 81.585 90)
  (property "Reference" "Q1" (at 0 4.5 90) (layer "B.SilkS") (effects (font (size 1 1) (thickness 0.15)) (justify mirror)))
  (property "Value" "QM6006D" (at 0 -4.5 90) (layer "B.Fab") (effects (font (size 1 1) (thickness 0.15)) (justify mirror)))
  (pad "" smd roundrect (at -0.415 -1.525 90) (size 3.05 2.75) (layers "B.Paste") (roundrect_rratio 0.090909))
  (pad "" smd roundrect (at -0.415 1.525 90) (size 3.05 2.75) (layers "B.Paste") (roundrect_rratio 0.090909))
  (pad "" smd roundrect (at 2.935 -1.525 90) (size 3.05 2.75) (layers "B.Paste") (roundrect_rratio 0.090909))
  (pad "" smd roundrect (at 2.935 1.525 90) (size 3.05 2.75) (layers "B.Paste") (roundrect_rratio 0.090909))
  (pad "1" smd roundrect (at -5.04 2.28 90) (size 2.2 1.2) (layers "B.Cu" "B.Mask" "B.Paste") (roundrect_rratio 0.208333) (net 2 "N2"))
  (pad "2" smd roundrect (at 1.26 0 90) (size 6.4 5.8) (layers "B.Cu" "B.Mask") (roundrect_rratio 0.043103) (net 8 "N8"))
  (pad "3" smd roundrect (at -5.04 -2.28 90) (size 2.2 1.2) (layers "B.Cu" "B.Mask" "B.Paste") (roundrect_rratio 0.208333) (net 3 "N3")))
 (gr_rect (start 108 76.5) (end 133 116.5) (stroke (width 0.05) (type default)) (fill no) (layer "Edge.Cuts"))
 (via (at 128 97.9) (size 0.6) (drill 0.3) (layers "F.Cu" "B.Cu") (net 8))
 (segment (start 128.026 97.874) (end 128 97.9) (width 0.2) (layer "B.Cu") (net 8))
 (segment (start 131.5 97.874) (end 128.026 97.874) (width 0.2) (layer "B.Cu") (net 8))
 (segment (start 132.251 83.601) (end 132.251 97.123) (width 0.2) (layer "B.Cu") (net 8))
 (segment (start 132.251 97.123) (end 131.5 97.874) (width 0.2) (layer "B.Cu") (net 8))
 (segment (start 128.975 80.325) (end 132.251 83.601) (width 0.2) (layer "B.Cu") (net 8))
 (via (at 128 95.1) (size 0.6) (drill 0.3) (layers "F.Cu" "B.Cu") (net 9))
 (segment (start 127.399 95.701) (end 128 95.1) (width 0.2) (layer "B.Cu") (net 9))
 (segment (start 127.399 99.399) (end 127.399 95.701) (width 0.2) (layer "B.Cu") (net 9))
 (segment (start 128 100) (end 127.399 99.399) (width 0.2) (layer "B.Cu") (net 9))
 (segment (start 115.9625 103.1375) (end 115.9625 103) (width 0.2) (layer "F.Cu") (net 11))
 (segment (start 113 106.1) (end 115.9625 103.1375) (width 0.2) (layer "F.Cu") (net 11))
 (via (at 115.9625 103) (size 0.6) (drill 0.3) (layers "F.Cu" "B.Cu") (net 11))
 (segment (start 125.55 108.9) (end 128.975 112.325) (width 0.2) (layer "F.Cu") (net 10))
 (segment (start 113 108.9) (end 125.55 108.9) (width 0.2) (layer "F.Cu") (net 10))
 (via (at 128.975 112.325) (size 0.6) (drill 0.3) (layers "F.Cu" "B.Cu") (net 10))
 (segment (start 113.5 88.5375) (end 113.0375 89) (width 0.2) (layer "F.Cu") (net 7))
 (segment (start 113.5 86.4) (end 113.5 88.5375) (width 0.2) (layer "F.Cu") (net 7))
 (via (at 113.0375 89) (size 0.6) (drill 0.3) (layers "F.Cu" "B.Cu") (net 7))
 (via (at 113.5 83.6) (size 0.6) (drill 0.3) (layers "F.Cu" "B.Cu") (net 6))
 (segment (start 116.86 80.24) (end 113.5 83.6) (width 0.2) (layer "B.Cu") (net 6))
 (segment (start 121.5 80.24) (end 116.86 80.24) (width 0.2) (layer "B.Cu") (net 6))
 (segment (start 109.9 104.975) (end 111.0625 104.975) (width 0.2) (layer "F.Cu") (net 1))
 (segment (start 113.0375 103) (end 113.521 102.5165) (width 0.2) (layer "F.Cu") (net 1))
 (segment (start 131.1 99.825) (end 128 102.925) (width 0.2) (layer "F.Cu") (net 1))
 (segment (start 113.521 96.021) (end 109.88 92.38) (width 0.2) (layer "F.Cu") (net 1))
 (segment (start 131.1 99.025) (end 131.1 99.825) (width 0.2) (layer "F.Cu") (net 1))
 (segment (start 111.0625 104.975) (end 113.0375 103) (width 0.2) (layer "F.Cu") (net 1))
 (segment (start 113.521 102.5165) (end 113.521 96.021) (width 0.2) (layer "F.Cu") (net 1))
 (via (at 128 102.925) (size 0.6) (drill 0.3) (layers "F.Cu" "B.Cu") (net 1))
 (via (at 113.0375 103) (size 0.6) (drill 0.3) (layers "F.Cu" "B.Cu") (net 1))
 (segment (start 108.849 91.349) (end 108.849 85.49176) (width 0.2) (layer "B.Cu") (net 1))
 (segment (start 126.749 104.176) (end 114.2135 104.176) (width 0.2) (layer "B.Cu") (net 1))
 (segment (start 113.1285 86.166) (end 115.9625 89) (width 0.2) (layer "B.Cu") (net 1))
 (segment (start 109.52324 86.166) (end 113.1285 86.166) (width 0.2) (layer "B.Cu") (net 1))
 (segment (start 108.849 85.49176) (end 109.52324 86.166) (width 0.2) (layer "B.Cu") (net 1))
 (segment (start 128 102.925) (end 126.749 104.176) (width 0.2) (layer "B.Cu") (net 1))
 (segment (start 109.88 92.38) (end 108.849 91.349) (width 0.2) (layer "B.Cu") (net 1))
 (segment (start 108.849 83.626) (end 108.849 85.49176) (width 0.2) (layer "B.Cu") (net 1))
 (segment (start 114.2135 104.176) (end 113.0375 103) (width 0.2) (layer "B.Cu") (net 1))
 (segment (start 110 82.475) (end 108.849 83.626) (width 0.2) (layer "B.Cu") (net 1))
 (segment (start 108.749 106.364) (end 108.749 103.671) (width 0.2) (layer "F.Cu") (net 4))
 (segment (start 109.9 107.515) (end 108.749 106.364) (width 0.2) (layer "F.Cu") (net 4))
 (segment (start 108.749 103.671) (end 112.42 100) (width 0.2) (layer "F.Cu") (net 4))
 (segment (start 126.695 106.025) (end 111.39 106.025) (width 0.2) (layer "B.Cu") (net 4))
 (segment (start 111.39 106.025) (end 109.9 107.515) (width 0.2) (layer "B.Cu") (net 4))
 (segment (start 125.12 100) (end 122.58 100) (width 0.2) (layer "F.Cu") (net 3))
 (segment (start 132.251 96.96176) (end 131.57676 97.636) (width 0.2) (layer "F.Cu") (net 3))
 (segment (start 130.62324 97.636) (end 129.548 96.56076) (width 0.2) (layer "F.Cu") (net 3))
 (segment (start 132.251 95.096) (end 132.251 105.029) (width 0.2) (layer "F.Cu") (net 3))
 (segment (start 129.548 94.86184) (end 127.06616 92.38) (width 0.2) (layer "F.Cu") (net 3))
 (segment (start 120.04 100) (end 117.5 100) (width 0.2) (layer "F.Cu") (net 3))
 (segment (start 132.251 105.029) (end 131.255 106.025) (width 0.2) (layer "F.Cu") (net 3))
 (segment (start 109.9 110.055) (end 112.929 107.026) (width 0.2) (layer "F.Cu") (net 3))
 (segment (start 112.929 107.026) (end 113.86016 107.026) (width 0.2) (layer "F.Cu") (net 3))
 (segment (start 131.1 93.945) (end 132.251 95.096) (width 0.2) (layer "F.Cu") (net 3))
 (segment (start 113.86016 107.026) (end 117.5 103.38616) (width 0.2) (layer "F.Cu") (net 3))
 (segment (start 127.06616 92.38) (end 125.12 92.38) (width 0.2) (layer "F.Cu") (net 3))
 (segment (start 132.251 95.096) (end 132.251 96.96176) (width 0.2) (layer "F.Cu") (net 3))
 (segment (start 122.58 100) (end 120.04 100) (width 0.2) (layer "F.Cu") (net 3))
 (segment (start 131.57676 97.636) (end 130.62324 97.636) (width 0.2) (layer "F.Cu") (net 3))
 (segment (start 129.548 96.56076) (end 129.548 94.86184) (width 0.2) (layer "F.Cu") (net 3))
 (segment (start 117.5 103.38616) (end 117.5 100) (width 0.2) (layer "F.Cu") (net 3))
 (via (at 131.255 106.025) (size 0.6) (drill 0.3) (layers "F.Cu" "B.Cu") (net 3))
 (segment (start 110 89.96) (end 110 87.555) (width 0.2) (layer "B.Cu") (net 3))
 (segment (start 125.12 92.38) (end 122.58 92.38) (width 0.2) (layer "B.Cu") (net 3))
 (segment (start 119.22 91.14) (end 119.22 86.54) (width 0.2) (layer "B.Cu") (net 3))
 (segment (start 125.9835 100.8635) (end 125.12 100) (width 0.2) (layer "B.Cu") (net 3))
 (segment (start 126.695 86.625) (end 126.695 90.805) (width 0.2) (layer "B.Cu") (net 3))
 (segment (start 126.695 90.805) (end 125.12 92.38) (width 0.2) (layer "B.Cu") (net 3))
 (segment (start 122.58 92.38) (end 120.04 92.38) (width 0.2) (layer "B.Cu") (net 3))
 (segment (start 128.3635 100.8635) (end 125.9835 100.8635) (width 0.2) (layer "B.Cu") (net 3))
 (segment (start 131.255 106.025) (end 131.255 103.755) (width 0.2) (layer "B.Cu") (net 3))
 (segment (start 131.255 103.755) (end 128.3635 100.8635) (width 0.2) (layer "B.Cu") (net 3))
 (segment (start 120.04 92.38) (end 117.5 92.38) (width 0.2) (layer "B.Cu") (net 3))
 (segment (start 112.42 92.38) (end 110 89.96) (width 0.2) (layer "B.Cu") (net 3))
 (segment (start 120.04 91.96) (end 119.22 91.14) (width 0.2) (layer "B.Cu") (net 3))
 (segment (start 114.96 92.38) (end 112.42 92.38) (width 0.2) (layer "B.Cu") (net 3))
 (segment (start 117.5 92.38) (end 114.96 92.38) (width 0.2) (layer "B.Cu") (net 3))
 (segment (start 120.04 92.38) (end 120.04 91.96) (width 0.2) (layer "B.Cu") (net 3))
 (segment (start 108.779 86.236) (end 110 85.015) (width 0.2) (layer "F.Cu") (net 2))
 (segment (start 109.88 100) (end 108.779 98.899) (width 0.2) (layer "F.Cu") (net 2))
 (segment (start 108.779 98.899) (end 108.779 86.236) (width 0.2) (layer "F.Cu") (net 2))
 (segment (start 131.255 86.625) (end 129.645 85.015) (width 0.2) (layer "B.Cu") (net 2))
 (segment (start 129.645 85.015) (end 110 85.015) (width 0.2) (layer "B.Cu") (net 2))
 (segment (start 126.56295 89.38) (end 126.62 89.38) (width 0.2) (layer "F.Cu") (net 5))
 (segment (start 129.949 95.334) (end 129.949 92.709) (width 0.2) (layer "F.Cu") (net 5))
 (segment (start 131.1 96.485) (end 129.949 95.334) (width 0.2) (layer "F.Cu") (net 5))
 (segment (start 114.96 100) (end 121.479 93.481) (width 0.2) (layer "F.Cu") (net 5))
 (segment (start 129.949 92.709) (end 126.62 89.38) (width 0.2) (layer "F.Cu") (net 5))
 (segment (start 123.37405 93.481) (end 124.019 92.83605) (width 0.2) (layer "F.Cu") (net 5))
 (segment (start 121.479 93.481) (end 123.37405 93.481) (width 0.2) (layer "F.Cu") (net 5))
 (segment (start 124.019 92.83605) (end 124.019 91.92395) (width 0.2) (layer "F.Cu") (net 5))
 (segment (start 124.019 91.92395) (end 126.56295 89.38) (width 0.2) (layer "F.Cu") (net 5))
 (segment (start 126.62 89.38) (end 123.78 86.54) (width 0.2) (layer "F.Cu") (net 5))
 (via (at 123.78 86.54) (size 0.6) (drill 0.3) (layers "F.Cu" "B.Cu") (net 5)))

